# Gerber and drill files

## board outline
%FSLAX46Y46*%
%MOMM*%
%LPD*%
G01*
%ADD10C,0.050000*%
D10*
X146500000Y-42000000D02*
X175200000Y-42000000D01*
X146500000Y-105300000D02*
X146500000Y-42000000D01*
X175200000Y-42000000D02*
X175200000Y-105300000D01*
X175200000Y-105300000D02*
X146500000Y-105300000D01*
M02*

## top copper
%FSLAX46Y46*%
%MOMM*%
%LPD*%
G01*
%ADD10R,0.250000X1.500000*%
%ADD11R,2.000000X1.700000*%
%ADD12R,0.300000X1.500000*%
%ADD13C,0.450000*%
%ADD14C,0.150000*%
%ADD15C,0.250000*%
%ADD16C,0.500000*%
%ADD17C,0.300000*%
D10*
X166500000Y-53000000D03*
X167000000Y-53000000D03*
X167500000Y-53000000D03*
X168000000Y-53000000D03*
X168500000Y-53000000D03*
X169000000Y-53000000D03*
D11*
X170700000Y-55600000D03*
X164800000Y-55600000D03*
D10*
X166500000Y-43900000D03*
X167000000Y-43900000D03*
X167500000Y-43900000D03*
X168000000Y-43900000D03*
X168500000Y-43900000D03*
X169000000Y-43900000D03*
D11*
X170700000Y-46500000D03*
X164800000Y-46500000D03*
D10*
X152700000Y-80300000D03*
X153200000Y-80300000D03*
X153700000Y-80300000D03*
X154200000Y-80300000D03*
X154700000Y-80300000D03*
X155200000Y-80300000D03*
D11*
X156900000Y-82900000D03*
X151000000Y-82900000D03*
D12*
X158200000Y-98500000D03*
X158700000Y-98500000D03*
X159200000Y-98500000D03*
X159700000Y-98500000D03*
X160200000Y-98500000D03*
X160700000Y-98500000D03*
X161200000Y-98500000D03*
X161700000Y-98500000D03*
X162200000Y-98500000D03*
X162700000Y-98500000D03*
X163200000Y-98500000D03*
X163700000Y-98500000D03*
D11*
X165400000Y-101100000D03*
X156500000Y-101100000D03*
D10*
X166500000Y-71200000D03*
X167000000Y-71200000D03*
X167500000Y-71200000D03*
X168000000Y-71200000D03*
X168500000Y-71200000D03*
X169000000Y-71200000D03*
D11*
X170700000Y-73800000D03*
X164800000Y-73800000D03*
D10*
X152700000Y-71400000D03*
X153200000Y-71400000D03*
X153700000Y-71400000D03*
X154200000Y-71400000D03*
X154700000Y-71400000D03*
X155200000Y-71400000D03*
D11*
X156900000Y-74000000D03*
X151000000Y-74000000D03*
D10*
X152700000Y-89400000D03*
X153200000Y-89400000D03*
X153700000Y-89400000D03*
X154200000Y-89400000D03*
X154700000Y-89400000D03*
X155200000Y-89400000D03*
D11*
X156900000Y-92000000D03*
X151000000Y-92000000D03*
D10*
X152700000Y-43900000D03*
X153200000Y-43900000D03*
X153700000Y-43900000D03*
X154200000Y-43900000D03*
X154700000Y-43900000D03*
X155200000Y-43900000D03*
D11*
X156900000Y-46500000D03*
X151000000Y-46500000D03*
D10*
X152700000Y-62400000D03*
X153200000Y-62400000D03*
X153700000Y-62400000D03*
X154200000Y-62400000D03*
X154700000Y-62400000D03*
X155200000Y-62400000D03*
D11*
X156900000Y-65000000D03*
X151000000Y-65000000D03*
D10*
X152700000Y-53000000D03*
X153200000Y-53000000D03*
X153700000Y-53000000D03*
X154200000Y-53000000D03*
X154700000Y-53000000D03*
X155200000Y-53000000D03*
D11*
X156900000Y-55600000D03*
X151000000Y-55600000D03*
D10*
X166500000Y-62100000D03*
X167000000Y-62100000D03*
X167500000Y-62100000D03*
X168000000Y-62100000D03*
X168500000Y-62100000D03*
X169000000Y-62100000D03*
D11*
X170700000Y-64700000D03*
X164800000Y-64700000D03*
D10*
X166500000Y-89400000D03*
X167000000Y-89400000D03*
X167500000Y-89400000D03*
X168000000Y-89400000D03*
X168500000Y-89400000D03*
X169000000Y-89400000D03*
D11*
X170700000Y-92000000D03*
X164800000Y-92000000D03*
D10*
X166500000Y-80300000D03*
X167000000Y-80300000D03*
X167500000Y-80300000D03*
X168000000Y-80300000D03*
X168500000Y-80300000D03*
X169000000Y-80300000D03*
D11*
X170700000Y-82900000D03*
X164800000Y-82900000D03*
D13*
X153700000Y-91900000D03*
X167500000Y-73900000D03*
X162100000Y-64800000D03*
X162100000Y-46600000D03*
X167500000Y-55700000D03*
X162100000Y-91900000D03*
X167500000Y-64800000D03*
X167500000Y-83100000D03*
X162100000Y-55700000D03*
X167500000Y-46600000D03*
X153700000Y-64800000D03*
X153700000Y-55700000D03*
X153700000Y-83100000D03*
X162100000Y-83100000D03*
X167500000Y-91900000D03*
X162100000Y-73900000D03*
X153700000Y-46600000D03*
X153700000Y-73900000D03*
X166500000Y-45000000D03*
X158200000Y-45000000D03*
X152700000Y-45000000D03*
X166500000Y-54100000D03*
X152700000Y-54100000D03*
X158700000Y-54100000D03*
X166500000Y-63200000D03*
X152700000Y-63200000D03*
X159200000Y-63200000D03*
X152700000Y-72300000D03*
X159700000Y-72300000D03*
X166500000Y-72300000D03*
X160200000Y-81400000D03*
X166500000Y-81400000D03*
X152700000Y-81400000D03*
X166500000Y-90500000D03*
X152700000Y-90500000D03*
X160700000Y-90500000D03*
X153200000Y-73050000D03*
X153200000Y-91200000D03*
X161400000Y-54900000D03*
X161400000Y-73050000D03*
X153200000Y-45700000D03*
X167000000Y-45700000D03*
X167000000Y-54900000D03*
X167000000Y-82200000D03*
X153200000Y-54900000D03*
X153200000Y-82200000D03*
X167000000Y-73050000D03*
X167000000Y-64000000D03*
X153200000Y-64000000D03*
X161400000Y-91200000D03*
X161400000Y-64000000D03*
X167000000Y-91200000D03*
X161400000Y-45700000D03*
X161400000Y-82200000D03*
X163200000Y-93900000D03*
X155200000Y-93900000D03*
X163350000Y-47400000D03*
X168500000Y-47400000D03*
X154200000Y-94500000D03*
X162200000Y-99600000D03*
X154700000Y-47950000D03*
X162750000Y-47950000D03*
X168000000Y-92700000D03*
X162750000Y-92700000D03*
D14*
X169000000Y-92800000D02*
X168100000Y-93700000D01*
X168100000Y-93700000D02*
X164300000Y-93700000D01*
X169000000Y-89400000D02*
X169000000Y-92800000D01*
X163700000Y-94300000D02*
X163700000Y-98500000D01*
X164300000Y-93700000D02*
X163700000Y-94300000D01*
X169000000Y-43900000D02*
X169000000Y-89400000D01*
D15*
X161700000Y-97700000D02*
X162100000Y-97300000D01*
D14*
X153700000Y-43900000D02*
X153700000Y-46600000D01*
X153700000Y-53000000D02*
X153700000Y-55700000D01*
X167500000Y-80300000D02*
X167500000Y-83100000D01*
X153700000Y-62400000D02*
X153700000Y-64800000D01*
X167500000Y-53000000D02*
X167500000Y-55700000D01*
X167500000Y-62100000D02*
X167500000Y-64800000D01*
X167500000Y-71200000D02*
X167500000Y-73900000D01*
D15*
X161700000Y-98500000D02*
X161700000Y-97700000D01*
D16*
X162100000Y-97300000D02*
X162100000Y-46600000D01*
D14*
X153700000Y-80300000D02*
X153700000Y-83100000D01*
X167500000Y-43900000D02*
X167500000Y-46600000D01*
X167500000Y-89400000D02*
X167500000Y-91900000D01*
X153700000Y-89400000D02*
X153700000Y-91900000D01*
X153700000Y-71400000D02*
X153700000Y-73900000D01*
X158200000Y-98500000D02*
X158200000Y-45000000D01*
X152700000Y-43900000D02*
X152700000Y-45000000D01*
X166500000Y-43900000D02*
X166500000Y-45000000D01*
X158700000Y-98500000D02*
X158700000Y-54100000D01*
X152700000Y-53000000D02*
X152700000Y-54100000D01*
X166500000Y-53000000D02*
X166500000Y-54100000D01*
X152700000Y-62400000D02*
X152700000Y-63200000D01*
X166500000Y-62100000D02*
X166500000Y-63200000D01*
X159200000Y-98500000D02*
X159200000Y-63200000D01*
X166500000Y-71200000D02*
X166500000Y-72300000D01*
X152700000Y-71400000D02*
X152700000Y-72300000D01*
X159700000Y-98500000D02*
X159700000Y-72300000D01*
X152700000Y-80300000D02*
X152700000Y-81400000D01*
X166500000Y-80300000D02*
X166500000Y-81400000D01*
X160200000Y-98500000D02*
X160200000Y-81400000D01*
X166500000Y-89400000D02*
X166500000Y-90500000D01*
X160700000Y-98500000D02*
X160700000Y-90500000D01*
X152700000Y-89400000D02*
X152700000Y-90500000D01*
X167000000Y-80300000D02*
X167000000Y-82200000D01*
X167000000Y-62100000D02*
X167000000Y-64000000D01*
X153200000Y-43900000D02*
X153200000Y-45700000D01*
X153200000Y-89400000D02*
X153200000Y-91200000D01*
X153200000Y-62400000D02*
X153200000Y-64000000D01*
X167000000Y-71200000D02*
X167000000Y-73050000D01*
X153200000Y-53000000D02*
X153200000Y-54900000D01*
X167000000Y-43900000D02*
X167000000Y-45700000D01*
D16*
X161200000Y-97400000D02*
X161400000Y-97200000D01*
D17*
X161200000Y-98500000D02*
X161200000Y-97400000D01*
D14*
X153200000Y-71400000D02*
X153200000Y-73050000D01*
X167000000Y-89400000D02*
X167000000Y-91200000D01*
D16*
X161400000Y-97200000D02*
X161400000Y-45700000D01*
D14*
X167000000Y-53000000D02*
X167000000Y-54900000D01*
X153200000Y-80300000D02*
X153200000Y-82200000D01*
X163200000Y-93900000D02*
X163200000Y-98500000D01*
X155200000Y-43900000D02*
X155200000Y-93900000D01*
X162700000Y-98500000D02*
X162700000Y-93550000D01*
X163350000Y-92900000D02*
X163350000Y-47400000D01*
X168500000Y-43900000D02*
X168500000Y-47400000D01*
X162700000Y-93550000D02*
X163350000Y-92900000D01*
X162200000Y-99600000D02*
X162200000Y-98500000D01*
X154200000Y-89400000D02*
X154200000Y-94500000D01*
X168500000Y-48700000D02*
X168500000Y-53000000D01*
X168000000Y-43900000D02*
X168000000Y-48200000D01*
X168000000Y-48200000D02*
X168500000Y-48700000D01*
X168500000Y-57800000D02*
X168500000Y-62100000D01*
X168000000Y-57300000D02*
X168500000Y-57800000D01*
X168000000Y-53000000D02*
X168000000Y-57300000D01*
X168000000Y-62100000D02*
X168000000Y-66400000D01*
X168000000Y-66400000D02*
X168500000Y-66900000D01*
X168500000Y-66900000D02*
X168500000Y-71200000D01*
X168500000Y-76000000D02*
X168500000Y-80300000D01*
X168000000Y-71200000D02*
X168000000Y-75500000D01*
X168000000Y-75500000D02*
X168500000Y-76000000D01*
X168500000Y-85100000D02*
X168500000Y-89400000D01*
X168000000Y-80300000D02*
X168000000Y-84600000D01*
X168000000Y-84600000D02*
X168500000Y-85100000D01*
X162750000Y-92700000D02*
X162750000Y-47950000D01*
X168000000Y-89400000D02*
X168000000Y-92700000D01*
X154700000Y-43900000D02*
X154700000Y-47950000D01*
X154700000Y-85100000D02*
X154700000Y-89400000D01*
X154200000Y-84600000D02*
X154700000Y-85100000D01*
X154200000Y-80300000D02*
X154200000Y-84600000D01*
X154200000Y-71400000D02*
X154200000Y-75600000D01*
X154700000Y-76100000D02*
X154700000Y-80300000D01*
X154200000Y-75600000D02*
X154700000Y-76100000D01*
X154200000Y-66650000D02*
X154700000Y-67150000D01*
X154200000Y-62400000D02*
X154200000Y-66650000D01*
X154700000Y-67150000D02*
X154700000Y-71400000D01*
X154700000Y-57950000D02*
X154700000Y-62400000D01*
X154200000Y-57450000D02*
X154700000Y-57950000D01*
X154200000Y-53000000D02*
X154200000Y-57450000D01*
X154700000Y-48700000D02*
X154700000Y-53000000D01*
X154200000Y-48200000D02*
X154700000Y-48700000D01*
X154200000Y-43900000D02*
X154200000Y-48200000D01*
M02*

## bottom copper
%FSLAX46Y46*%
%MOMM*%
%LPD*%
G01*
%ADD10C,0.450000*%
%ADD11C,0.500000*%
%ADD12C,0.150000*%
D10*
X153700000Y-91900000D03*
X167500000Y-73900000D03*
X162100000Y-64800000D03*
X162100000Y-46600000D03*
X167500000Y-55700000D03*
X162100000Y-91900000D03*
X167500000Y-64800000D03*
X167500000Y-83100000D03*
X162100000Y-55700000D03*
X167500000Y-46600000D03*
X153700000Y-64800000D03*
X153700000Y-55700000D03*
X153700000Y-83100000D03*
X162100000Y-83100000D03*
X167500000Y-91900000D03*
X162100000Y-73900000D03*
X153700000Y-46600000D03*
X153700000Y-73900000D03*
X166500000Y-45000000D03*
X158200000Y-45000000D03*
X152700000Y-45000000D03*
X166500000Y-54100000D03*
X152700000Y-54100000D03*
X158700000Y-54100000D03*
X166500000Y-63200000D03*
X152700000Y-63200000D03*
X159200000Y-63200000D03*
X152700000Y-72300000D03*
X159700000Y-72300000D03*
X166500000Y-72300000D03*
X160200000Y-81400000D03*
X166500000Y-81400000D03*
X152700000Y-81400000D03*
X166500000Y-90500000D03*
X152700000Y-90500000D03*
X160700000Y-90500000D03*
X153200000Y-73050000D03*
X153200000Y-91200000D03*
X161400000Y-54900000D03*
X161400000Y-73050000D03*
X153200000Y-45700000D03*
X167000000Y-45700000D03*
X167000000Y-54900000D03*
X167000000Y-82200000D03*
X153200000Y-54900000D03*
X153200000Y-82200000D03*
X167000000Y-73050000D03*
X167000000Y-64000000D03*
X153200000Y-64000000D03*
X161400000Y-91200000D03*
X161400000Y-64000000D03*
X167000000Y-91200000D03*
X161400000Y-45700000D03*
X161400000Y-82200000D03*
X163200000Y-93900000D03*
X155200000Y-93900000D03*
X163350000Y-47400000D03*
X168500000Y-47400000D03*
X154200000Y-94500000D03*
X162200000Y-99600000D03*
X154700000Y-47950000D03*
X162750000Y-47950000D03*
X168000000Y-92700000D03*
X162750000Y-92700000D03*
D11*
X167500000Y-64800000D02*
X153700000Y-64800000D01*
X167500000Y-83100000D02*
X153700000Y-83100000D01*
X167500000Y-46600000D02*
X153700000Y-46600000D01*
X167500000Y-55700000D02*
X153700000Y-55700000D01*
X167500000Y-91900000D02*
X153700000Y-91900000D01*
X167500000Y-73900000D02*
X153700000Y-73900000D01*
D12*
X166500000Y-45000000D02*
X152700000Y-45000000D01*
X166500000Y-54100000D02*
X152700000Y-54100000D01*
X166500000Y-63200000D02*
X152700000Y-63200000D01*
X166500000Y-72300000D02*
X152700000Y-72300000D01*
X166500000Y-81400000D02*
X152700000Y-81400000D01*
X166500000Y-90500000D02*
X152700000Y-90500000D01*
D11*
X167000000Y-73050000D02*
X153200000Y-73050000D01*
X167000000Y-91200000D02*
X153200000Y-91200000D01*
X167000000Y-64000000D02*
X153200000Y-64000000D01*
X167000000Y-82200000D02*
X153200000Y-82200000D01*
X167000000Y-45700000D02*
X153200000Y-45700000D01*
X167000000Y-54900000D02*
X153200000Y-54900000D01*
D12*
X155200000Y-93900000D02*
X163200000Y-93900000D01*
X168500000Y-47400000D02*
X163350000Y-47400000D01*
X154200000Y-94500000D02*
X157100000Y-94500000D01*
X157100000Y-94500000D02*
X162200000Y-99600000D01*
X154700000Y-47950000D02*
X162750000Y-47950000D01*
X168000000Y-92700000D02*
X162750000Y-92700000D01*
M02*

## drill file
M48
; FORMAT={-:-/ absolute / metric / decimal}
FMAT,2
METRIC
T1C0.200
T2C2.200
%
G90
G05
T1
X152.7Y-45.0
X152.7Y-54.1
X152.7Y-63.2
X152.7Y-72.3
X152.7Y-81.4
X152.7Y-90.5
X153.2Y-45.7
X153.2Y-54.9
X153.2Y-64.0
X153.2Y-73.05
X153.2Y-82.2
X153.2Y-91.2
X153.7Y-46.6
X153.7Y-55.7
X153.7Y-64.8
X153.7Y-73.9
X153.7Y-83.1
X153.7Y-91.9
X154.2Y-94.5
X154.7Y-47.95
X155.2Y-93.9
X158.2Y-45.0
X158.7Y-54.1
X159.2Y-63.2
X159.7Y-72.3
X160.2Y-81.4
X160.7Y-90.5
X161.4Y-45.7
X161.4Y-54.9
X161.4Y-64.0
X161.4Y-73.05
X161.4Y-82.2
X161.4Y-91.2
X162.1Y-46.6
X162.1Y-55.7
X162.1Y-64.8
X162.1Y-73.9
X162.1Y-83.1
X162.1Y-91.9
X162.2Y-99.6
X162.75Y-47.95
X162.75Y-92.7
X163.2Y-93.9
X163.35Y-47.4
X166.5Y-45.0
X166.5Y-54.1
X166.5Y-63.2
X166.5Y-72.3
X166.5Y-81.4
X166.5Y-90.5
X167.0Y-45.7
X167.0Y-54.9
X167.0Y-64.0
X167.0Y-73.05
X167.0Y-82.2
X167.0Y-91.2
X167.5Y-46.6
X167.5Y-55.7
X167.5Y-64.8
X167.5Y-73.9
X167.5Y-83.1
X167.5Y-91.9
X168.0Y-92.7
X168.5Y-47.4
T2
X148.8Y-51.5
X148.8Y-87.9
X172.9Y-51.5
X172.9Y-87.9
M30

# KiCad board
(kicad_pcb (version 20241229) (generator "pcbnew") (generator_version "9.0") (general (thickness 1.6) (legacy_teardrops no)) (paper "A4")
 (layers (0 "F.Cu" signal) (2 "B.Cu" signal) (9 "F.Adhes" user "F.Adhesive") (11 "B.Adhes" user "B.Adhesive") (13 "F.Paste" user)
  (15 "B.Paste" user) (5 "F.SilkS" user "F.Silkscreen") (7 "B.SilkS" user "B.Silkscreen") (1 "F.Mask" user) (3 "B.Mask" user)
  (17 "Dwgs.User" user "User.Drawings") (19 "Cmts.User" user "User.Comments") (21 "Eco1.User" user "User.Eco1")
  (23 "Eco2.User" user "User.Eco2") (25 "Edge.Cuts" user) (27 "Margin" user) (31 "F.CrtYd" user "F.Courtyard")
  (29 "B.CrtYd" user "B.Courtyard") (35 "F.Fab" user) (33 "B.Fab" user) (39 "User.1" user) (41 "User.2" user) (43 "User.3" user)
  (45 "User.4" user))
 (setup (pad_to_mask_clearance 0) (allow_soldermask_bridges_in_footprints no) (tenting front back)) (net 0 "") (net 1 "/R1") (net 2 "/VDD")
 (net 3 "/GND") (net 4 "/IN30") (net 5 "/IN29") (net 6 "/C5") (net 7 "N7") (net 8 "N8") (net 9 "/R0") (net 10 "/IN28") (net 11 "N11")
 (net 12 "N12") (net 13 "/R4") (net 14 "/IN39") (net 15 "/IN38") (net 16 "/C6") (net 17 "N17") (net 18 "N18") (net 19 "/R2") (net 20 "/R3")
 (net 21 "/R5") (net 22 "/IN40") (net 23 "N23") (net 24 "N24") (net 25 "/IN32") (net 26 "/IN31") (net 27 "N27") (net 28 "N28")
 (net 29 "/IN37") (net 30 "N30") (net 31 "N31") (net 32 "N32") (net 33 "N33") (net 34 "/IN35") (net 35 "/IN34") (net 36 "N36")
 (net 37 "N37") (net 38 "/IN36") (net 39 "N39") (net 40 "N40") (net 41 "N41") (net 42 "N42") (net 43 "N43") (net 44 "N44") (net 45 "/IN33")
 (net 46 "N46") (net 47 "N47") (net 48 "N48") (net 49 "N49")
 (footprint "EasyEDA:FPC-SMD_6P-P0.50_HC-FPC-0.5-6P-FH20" (layer "F.Cu") (at 167.75 54.3)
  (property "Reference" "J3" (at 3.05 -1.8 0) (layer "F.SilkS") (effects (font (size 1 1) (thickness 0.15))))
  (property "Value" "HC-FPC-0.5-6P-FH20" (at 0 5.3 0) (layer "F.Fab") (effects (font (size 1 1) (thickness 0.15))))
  (pad "1" smd rect (at -1.25 -1.3) (size 0.25 1.5) (layers "F.Cu" "F.Mask" "F.Paste") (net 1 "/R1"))
  (pad "2" smd rect (at -0.75 -1.3) (size 0.25 1.5) (layers "F.Cu" "F.Mask" "F.Paste") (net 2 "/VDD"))
  (pad "3" smd rect (at -0.25 -1.3) (size 0.25 1.5) (layers "F.Cu" "F.Mask" "F.Paste") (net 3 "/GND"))
  (pad "4" smd rect (at 0.25 -1.3) (size 0.25 1.5) (layers "F.Cu" "F.Mask" "F.Paste") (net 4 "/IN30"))
  (pad "5" smd rect (at 0.75 -1.3) (size 0.25 1.5) (layers "F.Cu" "F.Mask" "F.Paste") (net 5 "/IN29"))
  (pad "6" smd rect (at 1.25 -1.3) (size 0.25 1.5) (layers "F.Cu" "F.Mask" "F.Paste") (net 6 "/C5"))
  (pad "7" smd rect (at 2.95 1.3) (size 2 1.7) (layers "F.Cu" "F.Mask" "F.Paste") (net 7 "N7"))
  (pad "8" smd rect (at -2.95 1.3) (size 2 1.7) (layers "F.Cu" "F.Mask" "F.Paste") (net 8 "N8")))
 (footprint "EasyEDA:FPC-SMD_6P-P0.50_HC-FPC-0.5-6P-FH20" (layer "F.Cu") (at 167.75 45.2)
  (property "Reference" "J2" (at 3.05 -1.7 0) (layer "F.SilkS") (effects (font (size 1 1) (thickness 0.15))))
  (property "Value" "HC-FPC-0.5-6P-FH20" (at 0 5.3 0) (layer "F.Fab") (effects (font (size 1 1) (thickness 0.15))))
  (pad "1" smd rect (at -1.25 -1.3) (size 0.25 1.5) (layers "F.Cu" "F.Mask" "F.Paste") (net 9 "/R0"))
  (pad "2" smd rect (at -0.75 -1.3) (size 0.25 1.5) (layers "F.Cu" "F.Mask" "F.Paste") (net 2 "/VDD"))
  (pad "3" smd rect (at -0.25 -1.3) (size 0.25 1.5) (layers "F.Cu" "F.Mask" "F.Paste") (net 3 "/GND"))
  (pad "4" smd rect (at 0.25 -1.3) (size 0.25 1.5) (layers "F.Cu" "F.Mask" "F.Paste") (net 5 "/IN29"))
  (pad "5" smd rect (at 0.75 -1.3) (size 0.25 1.5) (layers "F.Cu" "F.Mask" "F.Paste") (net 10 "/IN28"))
  (pad "6" smd rect (at 1.25 -1.3) (size 0.25 1.5) (layers "F.Cu" "F.Mask" "F.Paste") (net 6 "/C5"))
  (pad "7" smd rect (at 2.95 1.3) (size 2 1.7) (layers "F.Cu" "F.Mask" "F.Paste") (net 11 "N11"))
  (pad "8" smd rect (at -2.95 1.3) (size 2 1.7) (layers "F.Cu" "F.Mask" "F.Paste") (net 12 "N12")))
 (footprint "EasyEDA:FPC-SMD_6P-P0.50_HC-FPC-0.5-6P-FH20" (layer "F.Cu") (at 153.95 81.6)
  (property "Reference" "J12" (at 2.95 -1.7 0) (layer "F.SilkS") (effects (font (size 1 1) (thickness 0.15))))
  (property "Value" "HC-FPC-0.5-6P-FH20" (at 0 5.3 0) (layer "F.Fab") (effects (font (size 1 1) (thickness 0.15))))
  (pad "1" smd rect (at -1.25 -1.3) (size 0.25 1.5) (layers "F.Cu" "F.Mask" "F.Paste") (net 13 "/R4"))
  (pad "2" smd rect (at -0.75 -1.3) (size 0.25 1.5) (layers "F.Cu" "F.Mask" "F.Paste") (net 2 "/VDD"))
  (pad "3" smd rect (at -0.25 -1.3) (size 0.25 1.5) (layers "F.Cu" "F.Mask" "F.Paste") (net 3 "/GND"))
  (pad "4" smd rect (at 0.25 -1.3) (size 0.25 1.5) (layers "F.Cu" "F.Mask" "F.Paste") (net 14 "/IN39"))
  (pad "5" smd rect (at 0.75 -1.3) (size 0.25 1.5) (layers "F.Cu" "F.Mask" "F.Paste") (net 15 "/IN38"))
  (pad "6" smd rect (at 1.25 -1.3) (size 0.25 1.5) (layers "F.Cu" "F.Mask" "F.Paste") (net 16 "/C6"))
  (pad "7" smd rect (at 2.95 1.3) (size 2 1.7) (layers "F.Cu" "F.Mask" "F.Paste") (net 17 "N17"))
  (pad "8" smd rect (at -2.95 1.3) (size 2 1.7) (layers "F.Cu" "F.Mask" "F.Paste") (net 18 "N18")))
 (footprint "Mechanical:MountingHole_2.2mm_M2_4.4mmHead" (layer "F.Cu") (at 148.8 87.9)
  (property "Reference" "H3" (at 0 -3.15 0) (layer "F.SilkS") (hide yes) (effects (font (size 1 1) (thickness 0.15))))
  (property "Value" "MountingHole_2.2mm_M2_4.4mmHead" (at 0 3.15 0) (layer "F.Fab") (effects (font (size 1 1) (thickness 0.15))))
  (pad "" np_thru_hole circle (at 0 0) (size 2.2 2.2) (drill 2.2) (layers "*.Cu" "*.Mask")))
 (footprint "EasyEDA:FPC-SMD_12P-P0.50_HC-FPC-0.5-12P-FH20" (layer "F.Cu") (at 160.95 99.8)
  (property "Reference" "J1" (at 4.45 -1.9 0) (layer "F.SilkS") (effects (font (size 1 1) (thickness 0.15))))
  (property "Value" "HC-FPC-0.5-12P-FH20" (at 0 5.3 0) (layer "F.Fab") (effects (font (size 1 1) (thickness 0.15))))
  (pad "1" smd rect (at -2.75 -1.3) (size 0.3 1.5) (layers "F.Cu" "F.Mask" "F.Paste") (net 9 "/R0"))
  (pad "2" smd rect (at -2.25 -1.3) (size 0.3 1.5) (layers "F.Cu" "F.Mask" "F.Paste") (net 1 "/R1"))
  (pad "3" smd rect (at -1.75 -1.3) (size 0.3 1.5) (layers "F.Cu" "F.Mask" "F.Paste") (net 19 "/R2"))
  (pad "4" smd rect (at -1.25 -1.3) (size 0.3 1.5) (layers "F.Cu" "F.Mask" "F.Paste") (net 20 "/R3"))
  (pad "5" smd rect (at -0.75 -1.3) (size 0.3 1.5) (layers "F.Cu" "F.Mask" "F.Paste") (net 13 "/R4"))
  (pad "6" smd rect (at -0.25 -1.3) (size 0.3 1.5) (layers "F.Cu" "F.Mask" "F.Paste") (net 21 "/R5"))
  (pad "7" smd rect (at 0.25 -1.3) (size 0.3 1.5) (layers "F.Cu" "F.Mask" "F.Paste") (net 2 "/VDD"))
  (pad "8" smd rect (at 0.75 -1.3) (size 0.3 1.5) (layers "F.Cu" "F.Mask" "F.Paste") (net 3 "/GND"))
  (pad "9" smd rect (at 1.25 -1.3) (size 0.3 1.5) (layers "F.Cu" "F.Mask" "F.Paste") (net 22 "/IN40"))
  (pad "10" smd rect (at 1.75 -1.3) (size 0.3 1.5) (layers "F.Cu" "F.Mask" "F.Paste") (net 10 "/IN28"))
  (pad "11" smd rect (at 2.25 -1.3) (size 0.3 1.5) (layers "F.Cu" "F.Mask" "F.Paste") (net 16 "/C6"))
  (pad "12" smd rect (at 2.75 -1.3) (size 0.3 1.5) (layers "F.Cu" "F.Mask" "F.Paste") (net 6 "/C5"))
  (pad "13" smd rect (at 4.45 1.3) (size 2 1.7) (layers "F.Cu" "F.Mask" "F.Paste") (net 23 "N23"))
  (pad "14" smd rect (at -4.45 1.3) (size 2 1.7) (layers "F.Cu" "F.Mask" "F.Paste") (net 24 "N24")))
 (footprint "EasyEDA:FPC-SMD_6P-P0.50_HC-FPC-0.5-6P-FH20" (layer "F.Cu") (at 167.75 72.5)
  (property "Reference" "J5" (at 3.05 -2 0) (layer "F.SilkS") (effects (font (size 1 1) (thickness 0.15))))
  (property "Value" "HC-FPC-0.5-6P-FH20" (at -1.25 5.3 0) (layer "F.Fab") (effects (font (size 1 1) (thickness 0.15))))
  (pad "1" smd rect (at -1.25 -1.3) (size 0.25 1.5) (layers "F.Cu" "F.Mask" "F.Paste") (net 20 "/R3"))
  (pad "2" smd rect (at -0.75 -1.3) (size 0.25 1.5) (layers "F.Cu" "F.Mask" "F.Paste") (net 2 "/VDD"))
  (pad "3" smd rect (at -0.25 -1.3) (size 0.25 1.5) (layers "F.Cu" "F.Mask" "F.Paste") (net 3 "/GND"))
  (pad "4" smd rect (at 0.25 -1.3) (size 0.25 1.5) (layers "F.Cu" "F.Mask" "F.Paste") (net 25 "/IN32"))
  (pad "5" smd rect (at 0.75 -1.3) (size 0.25 1.5) (layers "F.Cu" "F.Mask" "F.Paste") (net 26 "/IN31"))
  (pad "6" smd rect (at 1.25 -1.3) (size 0.25 1.5) (layers "F.Cu" "F.Mask" "F.Paste") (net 6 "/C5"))
  (pad "7" smd rect (at 2.95 1.3) (size 2 1.7) (layers "F.Cu" "F.Mask" "F.Paste") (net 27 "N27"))
  (pad "8" smd rect (at -2.95 1.3) (size 2 1.7) (layers "F.Cu" "F.Mask" "F.Paste") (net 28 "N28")))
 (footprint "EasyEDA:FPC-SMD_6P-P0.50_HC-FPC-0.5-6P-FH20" (layer "F.Cu") (at 153.95 72.7)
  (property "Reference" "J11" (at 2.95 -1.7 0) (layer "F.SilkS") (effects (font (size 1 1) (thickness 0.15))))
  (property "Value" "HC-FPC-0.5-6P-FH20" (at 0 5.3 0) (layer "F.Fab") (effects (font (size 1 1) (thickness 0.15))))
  (pad "1" smd rect (at -1.25 -1.3) (size 0.25 1.5) (layers "F.Cu" "F.Mask" "F.Paste") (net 20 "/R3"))
  (pad "2" smd rect (at -0.75 -1.3) (size 0.25 1.5) (layers "F.Cu" "F.Mask" "F.Paste") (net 2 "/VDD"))
  (pad "3" smd rect (at -0.25 -1.3) (size 0.25 1.5) (layers "F.Cu" "F.Mask" "F.Paste") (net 3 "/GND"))
  (pad "4" smd rect (at 0.25 -1.3) (size 0.25 1.5) (layers "F.Cu" "F.Mask" "F.Paste") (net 15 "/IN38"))
  (pad "5" smd rect (at 0.75 -1.3) (size 0.25 1.5) (layers "F.Cu" "F.Mask" "F.Paste") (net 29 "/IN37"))
  (pad "6" smd rect (at 1.25 -1.3) (size 0.25 1.5) (layers "F.Cu" "F.Mask" "F.Paste") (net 16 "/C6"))
  (pad "7" smd rect (at 2.95 1.3) (size 2 1.7) (layers "F.Cu" "F.Mask" "F.Paste") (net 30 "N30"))
  (pad "8" smd rect (at -2.95 1.3) (size 2 1.7) (layers "F.Cu" "F.Mask" "F.Paste") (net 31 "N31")))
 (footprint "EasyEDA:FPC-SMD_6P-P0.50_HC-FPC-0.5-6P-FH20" (layer "F.Cu") (at 153.95 90.7)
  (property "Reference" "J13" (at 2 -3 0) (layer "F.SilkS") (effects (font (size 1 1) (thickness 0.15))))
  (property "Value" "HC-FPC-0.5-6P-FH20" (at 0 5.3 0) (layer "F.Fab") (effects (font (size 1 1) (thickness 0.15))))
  (pad "1" smd rect (at -1.25 -1.3) (size 0.25 1.5) (layers "F.Cu" "F.Mask" "F.Paste") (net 21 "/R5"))
  (pad "2" smd rect (at -0.75 -1.3) (size 0.25 1.5) (layers "F.Cu" "F.Mask" "F.Paste") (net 2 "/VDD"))
  (pad "3" smd rect (at -0.25 -1.3) (size 0.25 1.5) (layers "F.Cu" "F.Mask" "F.Paste") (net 3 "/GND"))
  (pad "4" smd rect (at 0.25 -1.3) (size 0.25 1.5) (layers "F.Cu" "F.Mask" "F.Paste") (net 22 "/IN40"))
  (pad "5" smd rect (at 0.75 -1.3) (size 0.25 1.5) (layers "F.Cu" "F.Mask" "F.Paste") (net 14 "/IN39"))
  (pad "6" smd rect (at 1.25 -1.3) (size 0.25 1.5) (layers "F.Cu" "F.Mask" "F.Paste") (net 16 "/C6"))
  (pad "7" smd rect (at 2.95 1.3) (size 2 1.7) (layers "F.Cu" "F.Mask" "F.Paste") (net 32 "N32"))
  (pad "8" smd rect (at -2.95 1.3) (size 2 1.7) (layers "F.Cu" "F.Mask" "F.Paste") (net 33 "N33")))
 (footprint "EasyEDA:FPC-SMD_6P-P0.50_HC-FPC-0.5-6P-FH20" (layer "F.Cu") (at 153.95 45.2)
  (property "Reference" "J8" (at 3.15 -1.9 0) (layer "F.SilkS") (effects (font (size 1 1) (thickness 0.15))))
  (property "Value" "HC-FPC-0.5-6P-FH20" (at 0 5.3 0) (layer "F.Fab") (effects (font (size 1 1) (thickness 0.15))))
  (pad "1" smd rect (at -1.25 -1.3) (size 0.25 1.5) (layers "F.Cu" "F.Mask" "F.Paste") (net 9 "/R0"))
  (pad "2" smd rect (at -0.75 -1.3) (size 0.25 1.5) (layers "F.Cu" "F.Mask" "F.Paste") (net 2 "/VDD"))
  (pad "3" smd rect (at -0.25 -1.3) (size 0.25 1.5) (layers "F.Cu" "F.Mask" "F.Paste") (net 3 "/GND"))
  (pad "4" smd rect (at 0.25 -1.3) (size 0.25 1.5) (layers "F.Cu" "F.Mask" "F.Paste") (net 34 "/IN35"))
  (pad "5" smd rect (at 0.75 -1.3) (size 0.25 1.5) (layers "F.Cu" "F.Mask" "F.Paste") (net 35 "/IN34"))
  (pad "6" smd rect (at 1.25 -1.3) (size 0.25 1.5) (layers "F.Cu" "F.Mask" "F.Paste") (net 16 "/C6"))
  (pad "7" smd rect (at 2.95 1.3) (size 2 1.7) (layers "F.Cu" "F.Mask" "F.Paste") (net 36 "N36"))
  (pad "8" smd rect (at -2.95 1.3) (size 2 1.7) (layers "F.Cu" "F.Mask" "F.Paste") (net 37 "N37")))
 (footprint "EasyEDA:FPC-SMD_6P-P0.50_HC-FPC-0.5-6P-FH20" (layer "F.Cu") (at 153.95 63.7)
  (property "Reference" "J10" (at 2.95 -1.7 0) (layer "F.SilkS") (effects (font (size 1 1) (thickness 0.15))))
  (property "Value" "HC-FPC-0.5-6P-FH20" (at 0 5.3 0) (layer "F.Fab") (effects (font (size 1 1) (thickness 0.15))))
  (pad "1" smd rect (at -1.25 -1.3) (size 0.25 1.5) (layers "F.Cu" "F.Mask" "F.Paste") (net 19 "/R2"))
  (pad "2" smd rect (at -0.75 -1.3) (size 0.25 1.5) (layers "F.Cu" "F.Mask" "F.Paste") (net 2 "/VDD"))
  (pad "3" smd rect (at -0.25 -1.3) (size 0.25 1.5) (layers "F.Cu" "F.Mask" "F.Paste") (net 3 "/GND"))
  (pad "4" smd rect (at 0.25 -1.3) (size 0.25 1.5) (layers "F.Cu" "F.Mask" "F.Paste") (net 29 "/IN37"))
  (pad "5" smd rect (at 0.75 -1.3) (size 0.25 1.5) (layers "F.Cu" "F.Mask" "F.Paste") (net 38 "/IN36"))
  (pad "6" smd rect (at 1.25 -1.3) (size 0.25 1.5) (layers "F.Cu" "F.Mask" "F.Paste") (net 16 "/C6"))
  (pad "7" smd rect (at 2.95 1.3) (size 2 1.7) (layers "F.Cu" "F.Mask" "F.Paste") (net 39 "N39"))
  (pad "8" smd rect (at -2.95 1.3) (size 2 1.7) (layers "F.Cu" "F.Mask" "F.Paste") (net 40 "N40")))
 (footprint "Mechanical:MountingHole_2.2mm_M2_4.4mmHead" (layer "F.Cu") (at 172.9 51.5)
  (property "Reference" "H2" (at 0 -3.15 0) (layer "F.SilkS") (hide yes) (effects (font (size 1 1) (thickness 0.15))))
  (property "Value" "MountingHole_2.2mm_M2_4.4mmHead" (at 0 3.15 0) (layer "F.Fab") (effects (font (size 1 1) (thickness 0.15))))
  (pad "" np_thru_hole circle (at 0 0) (size 2.2 2.2) (drill 2.2) (layers "*.Cu" "*.Mask")))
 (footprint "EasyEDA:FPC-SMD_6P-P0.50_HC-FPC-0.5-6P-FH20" (layer "F.Cu") (at 153.95 54.3)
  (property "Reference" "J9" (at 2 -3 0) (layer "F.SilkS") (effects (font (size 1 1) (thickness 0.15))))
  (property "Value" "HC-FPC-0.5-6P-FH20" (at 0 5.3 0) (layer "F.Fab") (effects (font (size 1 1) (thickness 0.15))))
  (pad "1" smd rect (at -1.25 -1.3) (size 0.25 1.5) (layers "F.Cu" "F.Mask" "F.Paste") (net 1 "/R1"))
  (pad "2" smd rect (at -0.75 -1.3) (size 0.25 1.5) (layers "F.Cu" "F.Mask" "F.Paste") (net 2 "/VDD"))
  (pad "3" smd rect (at -0.25 -1.3) (size 0.25 1.5) (layers "F.Cu" "F.Mask" "F.Paste") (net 3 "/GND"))
  (pad "4" smd rect (at 0.25 -1.3) (size 0.25 1.5) (layers "F.Cu" "F.Mask" "F.Paste") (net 38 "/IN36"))
  (pad "5" smd rect (at 0.75 -1.3) (size 0.25 1.5) (layers "F.Cu" "F.Mask" "F.Paste") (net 34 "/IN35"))
  (pad "6" smd rect (at 1.25 -1.3) (size 0.25 1.5) (layers "F.Cu" "F.Mask" "F.Paste") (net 16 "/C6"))
  (pad "7" smd rect (at 2.95 1.3) (size 2 1.7) (layers "F.Cu" "F.Mask" "F.Paste") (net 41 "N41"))
  (pad "8" smd rect (at -2.95 1.3) (size 2 1.7) (layers "F.Cu" "F.Mask" "F.Paste") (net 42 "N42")))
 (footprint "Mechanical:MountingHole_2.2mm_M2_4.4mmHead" (layer "F.Cu") (at 148.8 51.5)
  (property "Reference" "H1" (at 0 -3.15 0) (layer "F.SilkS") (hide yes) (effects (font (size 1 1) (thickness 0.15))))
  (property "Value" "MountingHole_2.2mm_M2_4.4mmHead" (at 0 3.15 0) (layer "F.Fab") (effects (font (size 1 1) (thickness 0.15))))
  (pad "" np_thru_hole circle (at 0 0) (size 2.2 2.2) (drill 2.2) (layers "*.Cu" "*.Mask")))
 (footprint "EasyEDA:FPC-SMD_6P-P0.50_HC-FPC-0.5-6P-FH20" (layer "F.Cu") (at 167.75 63.4)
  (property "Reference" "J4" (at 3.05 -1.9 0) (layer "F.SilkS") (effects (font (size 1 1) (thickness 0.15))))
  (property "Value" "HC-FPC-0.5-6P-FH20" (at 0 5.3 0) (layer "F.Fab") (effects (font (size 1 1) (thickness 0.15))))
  (pad "1" smd rect (at -1.25 -1.3) (size 0.25 1.5) (layers "F.Cu" "F.Mask" "F.Paste") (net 19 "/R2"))
  (pad "2" smd rect (at -0.75 -1.3) (size 0.25 1.5) (layers "F.Cu" "F.Mask" "F.Paste") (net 2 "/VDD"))
  (pad "3" smd rect (at -0.25 -1.3) (size 0.25 1.5) (layers "F.Cu" "F.Mask" "F.Paste") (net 3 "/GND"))
  (pad "4" smd rect (at 0.25 -1.3) (size 0.25 1.5) (layers "F.Cu" "F.Mask" "F.Paste") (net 26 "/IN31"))
  (pad "5" smd rect (at 0.75 -1.3) (size 0.25 1.5) (layers "F.Cu" "F.Mask" "F.Paste") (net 4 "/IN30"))
  (pad "6" smd rect (at 1.25 -1.3) (size 0.25 1.5) (layers "F.Cu" "F.Mask" "F.Paste") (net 6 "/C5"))
  (pad "7" smd rect (at 2.95 1.3) (size 2 1.7) (layers "F.Cu" "F.Mask" "F.Paste") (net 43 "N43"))
  (pad "8" smd rect (at -2.95 1.3) (size 2 1.7) (layers "F.Cu" "F.Mask" "F.Paste") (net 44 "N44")))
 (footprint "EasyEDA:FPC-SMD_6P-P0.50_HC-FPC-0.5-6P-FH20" (layer "F.Cu") (at 167.75 90.7)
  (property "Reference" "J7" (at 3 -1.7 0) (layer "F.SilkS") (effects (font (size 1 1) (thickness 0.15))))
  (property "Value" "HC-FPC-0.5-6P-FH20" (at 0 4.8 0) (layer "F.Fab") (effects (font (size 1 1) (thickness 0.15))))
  (pad "1" smd rect (at -1.25 -1.3) (size 0.25 1.5) (layers "F.Cu" "F.Mask" "F.Paste") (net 21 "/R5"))
  (pad "2" smd rect (at -0.75 -1.3) (size 0.25 1.5) (layers "F.Cu" "F.Mask" "F.Paste") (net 2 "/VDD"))
  (pad "3" smd rect (at -0.25 -1.3) (size 0.25 1.5) (layers "F.Cu" "F.Mask" "F.Paste") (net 3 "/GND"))
  (pad "4" smd rect (at 0.25 -1.3) (size 0.25 1.5) (layers "F.Cu" "F.Mask" "F.Paste") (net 35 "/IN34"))
  (pad "5" smd rect (at 0.75 -1.3) (size 0.25 1.5) (layers "F.Cu" "F.Mask" "F.Paste") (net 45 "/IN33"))
  (pad "6" smd rect (at 1.25 -1.3) (size 0.25 1.5) (layers "F.Cu" "F.Mask" "F.Paste") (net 6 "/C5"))
  (pad "7" smd rect (at 2.95 1.3) (size 2 1.7) (layers "F.Cu" "F.Mask" "F.Paste") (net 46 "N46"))
  (pad "8" smd rect (at -2.95 1.3) (size 2 1.7) (layers "F.Cu" "F.Mask" "F.Paste") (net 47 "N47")))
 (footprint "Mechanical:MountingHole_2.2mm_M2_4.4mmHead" (layer "F.Cu") (at 172.9 87.9)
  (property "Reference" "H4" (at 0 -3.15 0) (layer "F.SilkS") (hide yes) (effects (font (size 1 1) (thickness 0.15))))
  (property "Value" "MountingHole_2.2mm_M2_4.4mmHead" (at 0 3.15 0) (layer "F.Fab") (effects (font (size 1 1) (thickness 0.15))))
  (pad "" np_thru_hole circle (at 0 0) (size 2.2 2.2) (drill 2.2) (layers "*.Cu" "*.Mask")))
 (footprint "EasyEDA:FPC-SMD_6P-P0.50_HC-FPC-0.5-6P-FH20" (layer "F.Cu") (at 167.75 81.6)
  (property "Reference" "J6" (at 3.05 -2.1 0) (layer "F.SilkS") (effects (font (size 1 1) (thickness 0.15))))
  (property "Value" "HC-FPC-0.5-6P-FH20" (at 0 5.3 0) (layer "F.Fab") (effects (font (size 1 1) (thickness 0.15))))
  (pad "1" smd rect (at -1.25 -1.3) (size 0.25 1.5) (layers "F.Cu" "F.Mask" "F.Paste") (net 13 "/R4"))
  (pad "2" smd rect (at -0.75 -1.3) (size 0.25 1.5) (layers "F.Cu" "F.Mask" "F.Paste") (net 2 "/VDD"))
  (pad "3" smd rect (at -0.25 -1.3) (size 0.25 1.5) (layers "F.Cu" "F.Mask" "F.Paste") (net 3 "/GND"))
  (pad "4" smd rect (at 0.25 -1.3) (size 0.25 1.5) (layers "F.Cu" "F.Mask" "F.Paste") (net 45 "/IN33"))
  (pad "5" smd rect (at 0.75 -1.3) (size 0.25 1.5) (layers "F.Cu" "F.Mask" "F.Paste") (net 25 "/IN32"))
  (pad "6" smd rect (at 1.25 -1.3) (size 0.25 1.5) (layers "F.Cu" "F.Mask" "F.Paste") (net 6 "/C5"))
  (pad "7" smd rect (at 2.95 1.3) (size 2 1.7) (layers "F.Cu" "F.Mask" "F.Paste") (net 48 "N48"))
  (pad "8" smd rect (at -2.95 1.3) (size 2 1.7) (layers "F.Cu" "F.Mask" "F.Paste") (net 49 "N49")))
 (gr_line (start 146.5 42) (end 175.2 42) (stroke (width 0.05) (type default)) (layer "Edge.Cuts"))
 (gr_line (start 146.5 105.3) (end 146.5 42) (stroke (width 0.05) (type default)) (layer "Edge.Cuts"))
 (gr_line (start 175.2 42) (end 175.2 105.3) (stroke (width 0.05) (type default)) (layer "Edge.Cuts"))
 (gr_line (start 175.2 105.3) (end 146.5 105.3) (stroke (width 0.05) (type default)) (layer "Edge.Cuts"))
 (segment (start 169 92.8) (end 168.1 93.7) (width 0.15) (layer "F.Cu") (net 6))
 (segment (start 168.1 93.7) (end 164.3 93.7) (width 0.15) (layer "F.Cu") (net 6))
 (segment (start 169 89.4) (end 169 92.8) (width 0.15) (layer "F.Cu") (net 6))
 (segment (start 163.7 94.3) (end 163.7 98.5) (width 0.15) (layer "F.Cu") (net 6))
 (segment (start 164.3 93.7) (end 163.7 94.3) (width 0.15) (layer "F.Cu") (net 6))
 (segment (start 169 43.9) (end 169 89.4) (width 0.15) (layer "F.Cu") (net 6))
 (segment (start 161.7 97.7) (end 162.1 97.3) (width 0.25) (layer "F.Cu") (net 3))
 (segment (start 153.7 43.9) (end 153.7 46.6) (width 0.15) (layer "F.Cu") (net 3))
 (segment (start 153.7 53) (end 153.7 55.7) (width 0.15) (layer "F.Cu") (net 3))
 (segment (start 167.5 80.3) (end 167.5 83.1) (width 0.15) (layer "F.Cu") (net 3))
 (segment (start 153.7 62.4) (end 153.7 64.8) (width 0.15) (layer "F.Cu") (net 3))
 (segment (start 167.5 53) (end 167.5 55.7) (width 0.15) (layer "F.Cu") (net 3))
 (segment (start 167.5 62.1) (end 167.5 64.8) (width 0.15) (layer "F.Cu") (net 3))
 (segment (start 167.5 71.2) (end 167.5 73.9) (width 0.15) (layer "F.Cu") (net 3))
 (segment (start 161.7 98.5) (end 161.7 97.7) (width 0.25) (layer "F.Cu") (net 3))
 (segment (start 162.1 97.3) (end 162.1 46.6) (width 0.5) (layer "F.Cu") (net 3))
 (segment (start 153.7 80.3) (end 153.7 83.1) (width 0.15) (layer "F.Cu") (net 3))
 (segment (start 167.5 43.9) (end 167.5 46.6) (width 0.15) (layer "F.Cu") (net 3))
 (segment (start 167.5 89.4) (end 167.5 91.9) (width 0.15) (layer "F.Cu") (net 3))
 (segment (start 153.7 89.4) (end 153.7 91.9) (width 0.15) (layer "F.Cu") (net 3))
 (segment (start 153.7 71.4) (end 153.7 73.9) (width 0.15) (layer "F.Cu") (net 3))
 (via (at 153.7 91.9) (size 0.45) (drill 0.2) (layers "F.Cu" "B.Cu") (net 3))
 (via (at 167.5 73.9) (size 0.45) (drill 0.2) (layers "F.Cu" "B.Cu") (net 3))
 (via (at 162.1 64.8) (size 0.45) (drill 0.2) (layers "F.Cu" "B.Cu") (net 3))
 (via (at 162.1 46.6) (size 0.45) (drill 0.2) (layers "F.Cu" "B.Cu") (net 3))
 (via (at 167.5 55.7) (size 0.45) (drill 0.2) (layers "F.Cu" "B.Cu") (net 3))
 (via (at 162.1 91.9) (size 0.45) (drill 0.2) (layers "F.Cu" "B.Cu") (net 3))
 (via (at 167.5 64.8) (size 0.45) (drill 0.2) (layers "F.Cu" "B.Cu") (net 3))
 (via (at 167.5 83.1) (size 0.45) (drill 0.2) (layers "F.Cu" "B.Cu") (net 3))
 (via (at 162.1 55.7) (size 0.45) (drill 0.2) (layers "F.Cu" "B.Cu") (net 3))
 (via (at 167.5 46.6) (size 0.45) (drill 0.2) (layers "F.Cu" "B.Cu") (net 3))
 (via (at 153.7 64.8) (size 0.45) (drill 0.2) (layers "F.Cu" "B.Cu") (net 3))
 (via (at 153.7 55.7) (size 0.45) (drill 0.2) (layers "F.Cu" "B.Cu") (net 3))
 (via (at 153.7 83.1) (size 0.45) (drill 0.2) (layers "F.Cu" "B.Cu") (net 3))
 (via (at 162.1 83.1) (size 0.45) (drill 0.2) (layers "F.Cu" "B.Cu") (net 3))
 (via (at 167.5 91.9) (size 0.45) (drill 0.2) (layers "F.Cu" "B.Cu") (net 3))
 (via (at 162.1 73.9) (size 0.45) (drill 0.2) (layers "F.Cu" "B.Cu") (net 3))
 (via (at 153.7 46.6) (size 0.45) (drill 0.2) (layers "F.Cu" "B.Cu") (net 3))
 (via (at 153.7 73.9) (size 0.45) (drill 0.2) (layers "F.Cu" "B.Cu") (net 3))
 (segment (start 167.5 64.8) (end 153.7 64.8) (width 0.5) (layer "B.Cu") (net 3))
 (segment (start 167.5 83.1) (end 153.7 83.1) (width 0.5) (layer "B.Cu") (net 3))
 (segment (start 167.5 46.6) (end 153.7 46.6) (width 0.5) (layer "B.Cu") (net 3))
 (segment (start 167.5 55.7) (end 153.7 55.7) (width 0.5) (layer "B.Cu") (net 3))
 (segment (start 167.5 91.9) (end 153.7 91.9) (width 0.5) (layer "B.Cu") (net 3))
 (segment (start 167.5 73.9) (end 153.7 73.9) (width 0.5) (layer "B.Cu") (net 3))
 (segment (start 158.2 98.5) (end 158.2 45) (width 0.15) (layer "F.Cu") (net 9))
 (segment (start 152.7 43.9) (end 152.7 45) (width 0.15) (layer "F.Cu") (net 9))
 (segment (start 166.5 43.9) (end 166.5 45) (width 0.15) (layer "F.Cu") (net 9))
 (via (at 166.5 45) (size 0.45) (drill 0.2) (layers "F.Cu" "B.Cu") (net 9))
 (via (at 158.2 45) (size 0.45) (drill 0.2) (layers "F.Cu" "B.Cu") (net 9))
 (via (at 152.7 45) (size 0.45) (drill 0.2) (layers "F.Cu" "B.Cu") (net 9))
 (segment (start 166.5 45) (end 152.7 45) (width 0.15) (layer "B.Cu") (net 9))
 (segment (start 158.7 98.5) (end 158.7 54.1) (width 0.15) (layer "F.Cu") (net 1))
 (segment (start 152.7 53) (end 152.7 54.1) (width 0.15) (layer "F.Cu") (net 1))
 (segment (start 166.5 53) (end 166.5 54.1) (width 0.15) (layer "F.Cu") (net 1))
 (via (at 166.5 54.1) (size 0.45) (drill 0.2) (layers "F.Cu" "B.Cu") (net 1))
 (via (at 152.7 54.1) (size 0.45) (drill 0.2) (layers "F.Cu" "B.Cu") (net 1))
 (via (at 158.7 54.1) (size 0.45) (drill 0.2) (layers "F.Cu" "B.Cu") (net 1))
 (segment (start 166.5 54.1) (end 152.7 54.1) (width 0.15) (layer "B.Cu") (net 1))
 (segment (start 152.7 62.4) (end 152.7 63.2) (width 0.15) (layer "F.Cu") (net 19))
 (segment (start 166.5 62.1) (end 166.5 63.2) (width 0.15) (layer "F.Cu") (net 19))
 (segment (start 159.2 98.5) (end 159.2 63.2) (width 0.15) (layer "F.Cu") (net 19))
 (via (at 166.5 63.2) (size 0.45) (drill 0.2) (layers "F.Cu" "B.Cu") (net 19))
 (via (at 152.7 63.2) (size 0.45) (drill 0.2) (layers "F.Cu" "B.Cu") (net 19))
 (via (at 159.2 63.2) (size 0.45) (drill 0.2) (layers "F.Cu" "B.Cu") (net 19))
 (segment (start 166.5 63.2) (end 152.7 63.2) (width 0.15) (layer "B.Cu") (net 19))
 (segment (start 166.5 71.2) (end 166.5 72.3) (width 0.15) (layer "F.Cu") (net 20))
 (segment (start 152.7 71.4) (end 152.7 72.3) (width 0.15) (layer "F.Cu") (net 20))
 (segment (start 159.7 98.5) (end 159.7 72.3) (width 0.15) (layer "F.Cu") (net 20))
 (via (at 152.7 72.3) (size 0.45) (drill 0.2) (layers "F.Cu" "B.Cu") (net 20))
 (via (at 159.7 72.3) (size 0.45) (drill 0.2) (layers "F.Cu" "B.Cu") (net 20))
 (via (at 166.5 72.3) (size 0.45) (drill 0.2) (layers "F.Cu" "B.Cu") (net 20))
 (segment (start 166.5 72.3) (end 152.7 72.3) (width 0.15) (layer "B.Cu") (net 20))
 (segment (start 152.7 80.3) (end 152.7 81.4) (width 0.15) (layer "F.Cu") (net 13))
 (segment (start 166.5 80.3) (end 166.5 81.4) (width 0.15) (layer "F.Cu") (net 13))
 (segment (start 160.2 98.5) (end 160.2 81.4) (width 0.15) (layer "F.Cu") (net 13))
 (via (at 160.2 81.4) (size 0.45) (drill 0.2) (layers "F.Cu" "B.Cu") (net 13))
 (via (at 166.5 81.4) (size 0.45) (drill 0.2) (layers "F.Cu" "B.Cu") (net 13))
 (via (at 152.7 81.4) (size 0.45) (drill 0.2) (layers "F.Cu" "B.Cu") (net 13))
 (segment (start 166.5 81.4) (end 152.7 81.4) (width 0.15) (layer "B.Cu") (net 13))
 (segment (start 166.5 89.4) (end 166.5 90.5) (width 0.15) (layer "F.Cu") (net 21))
 (segment (start 160.7 98.5) (end 160.7 90.5) (width 0.15) (layer "F.Cu") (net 21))
 (segment (start 152.7 89.4) (end 152.7 90.5) (width 0.15) (layer "F.Cu") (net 21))
 (via (at 166.5 90.5) (size 0.45) (drill 0.2) (layers "F.Cu" "B.Cu") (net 21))
 (via (at 152.7 90.5) (size 0.45) (drill 0.2) (layers "F.Cu" "B.Cu") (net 21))
 (via (at 160.7 90.5) (size 0.45) (drill 0.2) (layers "F.Cu" "B.Cu") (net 21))
 (segment (start 166.5 90.5) (end 152.7 90.5) (width 0.15) (layer "B.Cu") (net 21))
 (segment (start 167 80.3) (end 167 82.2) (width 0.15) (layer "F.Cu") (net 2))
 (segment (start 167 62.1) (end 167 64) (width 0.15) (layer "F.Cu") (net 2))
 (segment (start 153.2 43.9) (end 153.2 45.7) (width 0.15) (layer "F.Cu") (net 2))
 (segment (start 153.2 89.4) (end 153.2 91.2) (width 0.15) (layer "F.Cu") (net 2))
 (segment (start 153.2 62.4) (end 153.2 64) (width 0.15) (layer "F.Cu") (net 2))
 (segment (start 167 71.2) (end 167 73.05) (width 0.15) (layer "F.Cu") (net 2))
 (segment (start 153.2 53) (end 153.2 54.9) (width 0.15) (layer "F.Cu") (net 2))
 (segment (start 167 43.9) (end 167 45.7) (width 0.15) (layer "F.Cu") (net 2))
 (segment (start 161.2 97.4) (end 161.4 97.2) (width 0.5) (layer "F.Cu") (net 2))
 (segment (start 161.2 98.5) (end 161.2 97.4) (width 0.3) (layer "F.Cu") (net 2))
 (segment (start 153.2 71.4) (end 153.2 73.05) (width 0.15) (layer "F.Cu") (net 2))
 (segment (start 167 89.4) (end 167 91.2) (width 0.15) (layer "F.Cu") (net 2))
 (segment (start 161.4 97.2) (end 161.4 45.7) (width 0.5) (layer "F.Cu") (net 2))
 (segment (start 167 53) (end 167 54.9) (width 0.15) (layer "F.Cu") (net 2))
 (segment (start 153.2 80.3) (end 153.2 82.2) (width 0.15) (layer "F.Cu") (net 2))
 (via (at 153.2 73.05) (size 0.45) (drill 0.2) (layers "F.Cu" "B.Cu") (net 2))
 (via (at 153.2 91.2) (size 0.45) (drill 0.2) (layers "F.Cu" "B.Cu") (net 2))
 (via (at 161.4 54.9) (size 0.45) (drill 0.2) (layers "F.Cu" "B.Cu") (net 2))
 (via (at 161.4 73.05) (size 0.45) (drill 0.2) (layers "F.Cu" "B.Cu") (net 2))
 (via (at 153.2 45.7) (size 0.45) (drill 0.2) (layers "F.Cu" "B.Cu") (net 2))
 (via (at 167 45.7) (size 0.45) (drill 0.2) (layers "F.Cu" "B.Cu") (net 2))
 (via (at 167 54.9) (size 0.45) (drill 0.2) (layers "F.Cu" "B.Cu") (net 2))
 (via (at 167 82.2) (size 0.45) (drill 0.2) (layers "F.Cu" "B.Cu") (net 2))
 (via (at 153.2 54.9) (size 0.45) (drill 0.2) (layers "F.Cu" "B.Cu") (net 2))
 (via (at 153.2 82.2) (size 0.45) (drill 0.2) (layers "F.Cu" "B.Cu") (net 2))
 (via (at 167 73.05) (size 0.45) (drill 0.2) (layers "F.Cu" "B.Cu") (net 2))
 (via (at 167 64) (size 0.45) (drill 0.2) (layers "F.Cu" "B.Cu") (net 2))
 (via (at 153.2 64) (size 0.45) (drill 0.2) (layers "F.Cu" "B.Cu") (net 2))
 (via (at 161.4 91.2) (size 0.45) (drill 0.2) (layers "F.Cu" "B.Cu") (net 2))
 (via (at 161.4 64) (size 0.45) (drill 0.2) (layers "F.Cu" "B.Cu") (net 2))
 (via (at 167 91.2) (size 0.45) (drill 0.2) (layers "F.Cu" "B.Cu") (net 2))
 (via (at 161.4 45.7) (size 0.45) (drill 0.2) (layers "F.Cu" "B.Cu") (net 2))
 (via (at 161.4 82.2) (size 0.45) (drill 0.2) (layers "F.Cu" "B.Cu") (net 2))
 (segment (start 167 73.05) (end 153.2 73.05) (width 0.5) (layer "B.Cu") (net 2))
 (segment (start 167 91.2) (end 153.2 91.2) (width 0.5) (layer "B.Cu") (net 2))
 (segment (start 167 64) (end 153.2 64) (width 0.5) (layer "B.Cu") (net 2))
 (segment (start 167 82.2) (end 153.2 82.2) (width 0.5) (layer "B.Cu") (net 2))
 (segment (start 167 45.7) (end 153.2 45.7) (width 0.5) (layer "B.Cu") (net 2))
 (segment (start 167 54.9) (end 153.2 54.9) (width 0.5) (layer "B.Cu") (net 2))
 (segment (start 163.2 93.9) (end 163.2 98.5) (width 0.15) (layer "F.Cu") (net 16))
 (segment (start 155.2 43.9) (end 155.2 93.9) (width 0.15) (layer "F.Cu") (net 16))
 (via (at 163.2 93.9) (size 0.45) (drill 0.2) (layers "F.Cu" "B.Cu") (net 16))
 (via (at 155.2 93.9) (size 0.45) (drill 0.2) (layers "F.Cu" "B.Cu") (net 16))
 (segment (start 155.2 93.9) (end 163.2 93.9) (width 0.15) (layer "B.Cu") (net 16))
 (segment (start 162.7 98.5) (end 162.7 93.55) (width 0.15) (layer "F.Cu") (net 10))
 (segment (start 163.35 92.9) (end 163.35 47.4) (width 0.15) (layer "F.Cu") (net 10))
 (segment (start 168.5 43.9) (end 168.5 47.4) (width 0.15) (layer "F.Cu") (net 10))
 (segment (start 162.7 93.55) (end 163.35 92.9) (width 0.15) (layer "F.Cu") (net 10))
 (via (at 163.35 47.4) (size 0.45) (drill 0.2) (layers "F.Cu" "B.Cu") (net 10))
 (via (at 168.5 47.4) (size 0.45) (drill 0.2) (layers "F.Cu" "B.Cu") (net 10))
 (segment (start 168.5 47.4) (end 163.35 47.4) (width 0.15) (layer "B.Cu") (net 10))
 (segment (start 162.2 99.6) (end 162.2 98.5) (width 0.15) (layer "F.Cu") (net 22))
 (segment (start 154.2 89.4) (end 154.2 94.5) (width 0.15) (layer "F.Cu") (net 22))
 (via (at 154.2 94.5) (size 0.45) (drill 0.2) (layers "F.Cu" "B.Cu") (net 22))
 (via (at 162.2 99.6) (size 0.45) (drill 0.2) (layers "F.Cu" "B.Cu") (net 22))
 (segment (start 154.2 94.5) (end 157.1 94.5) (width 0.15) (layer "B.Cu") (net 22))
 (segment (start 157.1 94.5) (end 162.2 99.6) (width 0.15) (layer "B.Cu") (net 22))
 (segment (start 168.5 48.7) (end 168.5 53) (width 0.15) (layer "F.Cu") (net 5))
 (segment (start 168 43.9) (end 168 48.2) (width 0.15) (layer "F.Cu") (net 5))
 (segment (start 168 48.2) (end 168.5 48.7) (width 0.15) (layer "F.Cu") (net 5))
 (segment (start 168.5 57.8) (end 168.5 62.1) (width 0.15) (layer "F.Cu") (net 4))
 (segment (start 168 57.3) (end 168.5 57.8) (width 0.15) (layer "F.Cu") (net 4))
 (segment (start 168 53) (end 168 57.3) (width 0.15) (layer "F.Cu") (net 4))
 (segment (start 168 62.1) (end 168 66.4) (width 0.15) (layer "F.Cu") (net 26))
 (segment (start 168 66.4) (end 168.5 66.9) (width 0.15) (layer "F.Cu") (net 26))
 (segment (start 168.5 66.9) (end 168.5 71.2) (width 0.15) (layer "F.Cu") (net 26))
 (segment (start 168.5 76) (end 168.5 80.3) (width 0.15) (layer "F.Cu") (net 25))
 (segment (start 168 71.2) (end 168 75.5) (width 0.15) (layer "F.Cu") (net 25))
 (segment (start 168 75.5) (end 168.5 76) (width 0.15) (layer "F.Cu") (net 25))
 (segment (start 168.5 85.1) (end 168.5 89.4) (width 0.15) (layer "F.Cu") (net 45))
 (segment (start 168 80.3) (end 168 84.6) (width 0.15) (layer "F.Cu") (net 45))
 (segment (start 168 84.6) (end 168.5 85.1) (width 0.15) (layer "F.Cu") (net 45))
 (segment (start 162.75 92.7) (end 162.75 47.95) (width 0.15) (layer "F.Cu") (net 35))
 (segment (start 168 89.4) (end 168 92.7) (width 0.15) (layer "F.Cu") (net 35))
 (segment (start 154.7 43.9) (end 154.7 47.95) (width 0.15) (layer "F.Cu") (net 35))
 (via (at 154.7 47.95) (size 0.45) (drill 0.2) (layers "F.Cu" "B.Cu") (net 35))
 (via (at 162.75 47.95) (size 0.45) (drill 0.2) (layers "F.Cu" "B.Cu") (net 35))
 (via (at 168 92.7) (size 0.45) (drill 0.2) (layers "F.Cu" "B.Cu") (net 35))
 (via (at 162.75 92.7) (size 0.45) (drill 0.2) (layers "F.Cu" "B.Cu") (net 35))
 (segment (start 154.7 47.95) (end 162.75 47.95) (width 0.15) (layer "B.Cu") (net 35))
 (segment (start 168 92.7) (end 162.75 92.7) (width 0.15) (layer "B.Cu") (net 35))
 (segment (start 154.7 85.1) (end 154.7 89.4) (width 0.15) (layer "F.Cu") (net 14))
 (segment (start 154.2 84.6) (end 154.7 85.1) (width 0.15) (layer "F.Cu") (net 14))
 (segment (start 154.2 80.3) (end 154.2 84.6) (width 0.15) (layer "F.Cu") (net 14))
 (segment (start 154.2 71.4) (end 154.2 75.6) (width 0.15) (layer "F.Cu") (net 15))
 (segment (start 154.7 76.1) (end 154.7 80.3) (width 0.15) (layer "F.Cu") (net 15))
 (segment (start 154.2 75.6) (end 154.7 76.1) (width 0.15) (layer "F.Cu") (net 15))
 (segment (start 154.2 66.65) (end 154.7 67.15) (width 0.15) (layer "F.Cu") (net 29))
 (segment (start 154.2 62.4) (end 154.2 66.65) (width 0.15) (layer "F.Cu") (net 29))
 (segment (start 154.7 67.15) (end 154.7 71.4) (width 0.15) (layer "F.Cu") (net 29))
 (segment (start 154.7 57.95) (end 154.7 62.4) (width 0.15) (layer "F.Cu") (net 38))
 (segment (start 154.2 57.45) (end 154.7 57.95) (width 0.15) (layer "F.Cu") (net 38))
 (segment (start 154.2 53) (end 154.2 57.45) (width 0.15) (layer "F.Cu") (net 38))
 (segment (start 154.7 48.7) (end 154.7 53) (width 0.15) (layer "F.Cu") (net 34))
 (segment (start 154.2 48.2) (end 154.7 48.7) (width 0.15) (layer "F.Cu") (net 34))
 (segment (start 154.2 43.9) (end 154.2 48.2) (width 0.15) (layer "F.Cu") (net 34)))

